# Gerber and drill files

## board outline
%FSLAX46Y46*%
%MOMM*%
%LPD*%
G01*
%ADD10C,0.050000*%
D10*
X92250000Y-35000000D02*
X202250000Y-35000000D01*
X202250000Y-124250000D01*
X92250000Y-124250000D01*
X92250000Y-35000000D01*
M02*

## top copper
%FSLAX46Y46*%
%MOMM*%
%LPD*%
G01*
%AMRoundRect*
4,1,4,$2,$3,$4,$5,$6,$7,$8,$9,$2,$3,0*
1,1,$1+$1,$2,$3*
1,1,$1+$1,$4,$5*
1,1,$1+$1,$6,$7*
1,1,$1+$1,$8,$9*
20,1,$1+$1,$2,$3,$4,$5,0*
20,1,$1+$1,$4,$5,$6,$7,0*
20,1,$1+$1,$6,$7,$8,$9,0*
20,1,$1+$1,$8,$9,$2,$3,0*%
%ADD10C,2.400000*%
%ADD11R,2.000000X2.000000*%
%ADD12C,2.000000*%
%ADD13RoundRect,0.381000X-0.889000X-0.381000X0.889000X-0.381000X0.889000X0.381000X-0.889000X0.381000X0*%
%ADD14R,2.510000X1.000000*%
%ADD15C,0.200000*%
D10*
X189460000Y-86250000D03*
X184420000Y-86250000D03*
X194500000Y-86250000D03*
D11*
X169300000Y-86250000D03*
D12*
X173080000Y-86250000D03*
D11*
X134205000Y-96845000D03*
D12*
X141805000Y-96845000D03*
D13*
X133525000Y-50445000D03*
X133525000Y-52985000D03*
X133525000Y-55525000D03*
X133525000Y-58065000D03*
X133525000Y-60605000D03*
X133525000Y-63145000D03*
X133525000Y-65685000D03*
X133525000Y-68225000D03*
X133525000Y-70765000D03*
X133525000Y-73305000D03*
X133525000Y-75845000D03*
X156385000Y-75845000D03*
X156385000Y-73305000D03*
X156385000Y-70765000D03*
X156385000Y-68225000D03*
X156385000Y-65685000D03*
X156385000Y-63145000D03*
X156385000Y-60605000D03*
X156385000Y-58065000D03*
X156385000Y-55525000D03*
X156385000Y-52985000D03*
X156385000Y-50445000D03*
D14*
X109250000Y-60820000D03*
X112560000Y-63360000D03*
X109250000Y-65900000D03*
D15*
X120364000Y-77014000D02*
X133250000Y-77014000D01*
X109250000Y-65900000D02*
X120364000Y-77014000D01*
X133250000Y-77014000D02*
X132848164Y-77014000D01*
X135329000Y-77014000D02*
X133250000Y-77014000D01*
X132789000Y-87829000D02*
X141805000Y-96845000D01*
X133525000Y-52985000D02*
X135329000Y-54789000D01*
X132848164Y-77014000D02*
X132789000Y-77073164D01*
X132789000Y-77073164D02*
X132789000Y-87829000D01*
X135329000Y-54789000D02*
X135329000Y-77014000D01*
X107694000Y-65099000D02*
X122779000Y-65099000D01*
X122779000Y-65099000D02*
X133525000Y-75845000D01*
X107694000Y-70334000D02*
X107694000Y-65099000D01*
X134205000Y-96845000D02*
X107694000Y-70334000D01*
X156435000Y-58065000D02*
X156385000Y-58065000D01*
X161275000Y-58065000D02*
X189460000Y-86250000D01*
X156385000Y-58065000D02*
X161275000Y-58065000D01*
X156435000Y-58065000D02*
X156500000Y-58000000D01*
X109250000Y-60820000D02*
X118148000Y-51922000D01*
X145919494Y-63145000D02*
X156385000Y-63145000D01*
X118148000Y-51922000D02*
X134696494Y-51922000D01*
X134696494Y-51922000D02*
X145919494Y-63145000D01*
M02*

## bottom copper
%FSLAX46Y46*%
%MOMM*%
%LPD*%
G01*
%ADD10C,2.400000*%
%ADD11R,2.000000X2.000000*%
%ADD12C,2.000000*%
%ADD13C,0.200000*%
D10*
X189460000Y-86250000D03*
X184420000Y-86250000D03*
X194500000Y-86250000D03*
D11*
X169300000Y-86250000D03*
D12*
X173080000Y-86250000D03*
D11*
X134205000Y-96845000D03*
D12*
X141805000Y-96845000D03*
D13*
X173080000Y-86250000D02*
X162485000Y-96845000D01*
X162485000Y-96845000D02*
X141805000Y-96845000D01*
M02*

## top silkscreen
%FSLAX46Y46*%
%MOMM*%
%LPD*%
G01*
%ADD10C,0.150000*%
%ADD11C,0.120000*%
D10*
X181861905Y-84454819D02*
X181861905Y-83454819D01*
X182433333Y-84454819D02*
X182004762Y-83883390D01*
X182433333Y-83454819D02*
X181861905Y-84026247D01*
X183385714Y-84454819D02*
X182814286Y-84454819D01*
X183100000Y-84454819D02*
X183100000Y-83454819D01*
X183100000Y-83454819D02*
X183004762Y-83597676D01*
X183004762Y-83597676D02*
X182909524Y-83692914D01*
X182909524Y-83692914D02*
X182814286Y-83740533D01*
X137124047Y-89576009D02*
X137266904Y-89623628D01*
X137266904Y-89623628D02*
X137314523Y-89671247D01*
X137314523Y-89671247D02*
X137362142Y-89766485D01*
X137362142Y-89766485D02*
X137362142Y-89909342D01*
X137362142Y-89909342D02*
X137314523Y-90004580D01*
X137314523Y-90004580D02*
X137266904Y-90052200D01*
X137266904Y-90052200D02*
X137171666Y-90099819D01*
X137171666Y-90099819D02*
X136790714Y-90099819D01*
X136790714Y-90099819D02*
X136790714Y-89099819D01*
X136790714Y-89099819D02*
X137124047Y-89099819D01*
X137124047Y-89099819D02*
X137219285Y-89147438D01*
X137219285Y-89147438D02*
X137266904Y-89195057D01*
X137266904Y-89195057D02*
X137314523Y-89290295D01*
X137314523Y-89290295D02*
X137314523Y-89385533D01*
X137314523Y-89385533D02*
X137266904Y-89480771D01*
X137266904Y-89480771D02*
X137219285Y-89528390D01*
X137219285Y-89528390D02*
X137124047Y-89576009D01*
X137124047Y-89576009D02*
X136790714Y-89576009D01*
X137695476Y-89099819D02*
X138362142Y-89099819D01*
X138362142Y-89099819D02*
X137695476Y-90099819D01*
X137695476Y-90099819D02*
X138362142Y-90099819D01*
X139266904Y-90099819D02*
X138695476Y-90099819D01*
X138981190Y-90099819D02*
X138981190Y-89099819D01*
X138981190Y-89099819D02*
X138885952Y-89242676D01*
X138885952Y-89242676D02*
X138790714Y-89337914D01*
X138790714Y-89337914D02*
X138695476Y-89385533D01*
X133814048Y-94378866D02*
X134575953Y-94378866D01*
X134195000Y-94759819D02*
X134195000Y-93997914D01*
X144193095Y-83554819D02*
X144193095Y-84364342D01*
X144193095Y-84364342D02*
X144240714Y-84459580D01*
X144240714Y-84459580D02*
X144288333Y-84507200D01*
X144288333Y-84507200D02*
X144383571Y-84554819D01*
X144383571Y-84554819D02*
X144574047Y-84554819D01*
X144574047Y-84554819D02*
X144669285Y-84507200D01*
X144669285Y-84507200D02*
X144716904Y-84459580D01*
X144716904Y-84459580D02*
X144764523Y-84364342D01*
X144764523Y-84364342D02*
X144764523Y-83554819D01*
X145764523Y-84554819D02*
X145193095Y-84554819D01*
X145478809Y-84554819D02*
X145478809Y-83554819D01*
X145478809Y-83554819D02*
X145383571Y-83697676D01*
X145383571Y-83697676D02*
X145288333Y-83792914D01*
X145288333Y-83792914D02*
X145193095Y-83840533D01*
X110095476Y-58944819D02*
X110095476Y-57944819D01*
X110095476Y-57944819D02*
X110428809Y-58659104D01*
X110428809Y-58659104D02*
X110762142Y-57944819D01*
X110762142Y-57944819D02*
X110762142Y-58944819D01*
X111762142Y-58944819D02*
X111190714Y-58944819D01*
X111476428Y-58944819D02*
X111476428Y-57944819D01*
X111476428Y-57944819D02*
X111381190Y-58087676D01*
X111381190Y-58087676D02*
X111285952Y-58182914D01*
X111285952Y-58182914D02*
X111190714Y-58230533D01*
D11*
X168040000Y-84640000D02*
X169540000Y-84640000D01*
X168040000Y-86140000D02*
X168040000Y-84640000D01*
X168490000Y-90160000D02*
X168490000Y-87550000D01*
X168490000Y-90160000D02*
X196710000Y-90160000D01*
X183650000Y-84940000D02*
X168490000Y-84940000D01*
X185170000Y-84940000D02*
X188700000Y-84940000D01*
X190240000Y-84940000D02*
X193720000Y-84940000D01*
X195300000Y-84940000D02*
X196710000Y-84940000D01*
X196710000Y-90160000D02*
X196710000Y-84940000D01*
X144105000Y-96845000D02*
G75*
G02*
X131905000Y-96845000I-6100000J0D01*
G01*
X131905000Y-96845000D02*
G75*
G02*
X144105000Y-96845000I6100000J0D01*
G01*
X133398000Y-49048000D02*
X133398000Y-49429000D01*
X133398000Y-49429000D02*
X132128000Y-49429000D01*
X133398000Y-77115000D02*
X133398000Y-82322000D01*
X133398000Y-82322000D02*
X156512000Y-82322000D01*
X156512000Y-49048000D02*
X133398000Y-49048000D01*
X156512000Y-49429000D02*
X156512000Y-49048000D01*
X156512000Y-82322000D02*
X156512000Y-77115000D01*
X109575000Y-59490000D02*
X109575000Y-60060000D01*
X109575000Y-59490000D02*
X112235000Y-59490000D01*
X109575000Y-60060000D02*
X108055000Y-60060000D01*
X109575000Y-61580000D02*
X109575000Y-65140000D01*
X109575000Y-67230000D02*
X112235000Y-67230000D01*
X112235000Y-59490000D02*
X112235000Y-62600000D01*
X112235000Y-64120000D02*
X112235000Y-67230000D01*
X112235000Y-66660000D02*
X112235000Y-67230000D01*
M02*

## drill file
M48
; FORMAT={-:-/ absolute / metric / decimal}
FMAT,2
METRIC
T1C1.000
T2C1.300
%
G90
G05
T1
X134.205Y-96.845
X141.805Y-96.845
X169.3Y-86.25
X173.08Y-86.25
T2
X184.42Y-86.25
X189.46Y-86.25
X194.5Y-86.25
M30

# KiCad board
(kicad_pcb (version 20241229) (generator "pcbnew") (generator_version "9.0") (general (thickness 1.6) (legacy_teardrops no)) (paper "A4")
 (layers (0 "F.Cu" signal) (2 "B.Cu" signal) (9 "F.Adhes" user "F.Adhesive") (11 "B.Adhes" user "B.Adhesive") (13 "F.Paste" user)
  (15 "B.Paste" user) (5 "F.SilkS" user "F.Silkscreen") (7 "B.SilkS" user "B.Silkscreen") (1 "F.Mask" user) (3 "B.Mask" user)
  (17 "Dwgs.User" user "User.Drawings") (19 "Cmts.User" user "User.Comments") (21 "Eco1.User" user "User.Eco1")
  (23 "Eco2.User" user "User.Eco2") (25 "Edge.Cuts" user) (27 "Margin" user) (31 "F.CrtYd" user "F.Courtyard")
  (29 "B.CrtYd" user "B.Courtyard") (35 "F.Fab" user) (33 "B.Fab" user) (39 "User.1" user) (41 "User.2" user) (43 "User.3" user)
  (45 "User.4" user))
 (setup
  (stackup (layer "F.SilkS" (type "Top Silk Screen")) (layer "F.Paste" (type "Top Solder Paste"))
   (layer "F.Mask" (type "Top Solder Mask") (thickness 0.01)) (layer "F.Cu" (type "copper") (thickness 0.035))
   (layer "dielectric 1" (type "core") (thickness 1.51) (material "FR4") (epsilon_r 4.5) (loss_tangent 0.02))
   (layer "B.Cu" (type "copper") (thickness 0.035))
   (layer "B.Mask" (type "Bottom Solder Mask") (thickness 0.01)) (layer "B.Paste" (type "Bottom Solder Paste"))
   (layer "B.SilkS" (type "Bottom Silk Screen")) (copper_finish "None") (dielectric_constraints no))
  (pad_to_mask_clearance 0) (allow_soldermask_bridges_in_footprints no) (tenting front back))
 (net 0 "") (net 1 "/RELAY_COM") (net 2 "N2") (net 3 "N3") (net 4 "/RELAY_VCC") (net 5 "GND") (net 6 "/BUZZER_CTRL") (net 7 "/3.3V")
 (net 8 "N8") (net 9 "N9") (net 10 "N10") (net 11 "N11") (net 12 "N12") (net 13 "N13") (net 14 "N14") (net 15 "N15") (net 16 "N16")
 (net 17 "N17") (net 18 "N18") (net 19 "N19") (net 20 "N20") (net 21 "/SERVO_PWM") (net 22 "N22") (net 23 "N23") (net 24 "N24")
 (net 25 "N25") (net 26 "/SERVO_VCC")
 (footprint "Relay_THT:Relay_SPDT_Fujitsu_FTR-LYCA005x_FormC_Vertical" (layer "F.Cu") (at 169.3 86.25)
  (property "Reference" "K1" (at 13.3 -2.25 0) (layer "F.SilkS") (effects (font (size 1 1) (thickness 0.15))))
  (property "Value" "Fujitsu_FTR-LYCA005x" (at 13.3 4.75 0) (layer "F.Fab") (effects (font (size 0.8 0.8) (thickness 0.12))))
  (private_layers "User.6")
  (fp_line (start -1.26 -1.61) (end 0.24 -1.61) (stroke (width 0.12) (type solid)) (layer "F.SilkS"))
  (fp_line (start -1.26 -0.11) (end -1.26 -1.61) (stroke (width 0.12) (type solid)) (layer "F.SilkS"))
  (fp_line (start -0.81 3.91) (end -0.81 1.3) (stroke (width 0.12) (type solid)) (layer "F.SilkS"))
  (fp_line (start -0.81 3.91) (end 27.41 3.91) (stroke (width 0.12) (type solid)) (layer "F.SilkS"))
  (fp_line (start 14.35 -1.31) (end -0.81 -1.31) (stroke (width 0.12) (type solid)) (layer "F.SilkS"))
  (fp_line (start 15.87 -1.31) (end 19.4 -1.31) (stroke (width 0.12) (type solid)) (layer "F.SilkS"))
  (fp_line (start 20.94 -1.31) (end 24.42 -1.31) (stroke (width 0.12) (type solid)) (layer "F.SilkS"))
  (fp_line (start 26 -1.31) (end 27.41 -1.31) (stroke (width 0.12) (type solid)) (layer "F.SilkS"))
  (fp_line (start 27.41 3.91) (end 27.41 -1.31) (stroke (width 0.12) (type solid)) (layer "F.SilkS"))
  (pad "11" thru_hole circle (at 20.16 0) (size 2.4 2.4) (drill 1.3) (layers "*.Cu" "*.Mask") (remove_unused_layers no) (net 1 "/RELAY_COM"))
  (pad "12" thru_hole circle (at 15.12 0) (size 2.4 2.4) (drill 1.3) (layers "*.Cu" "*.Mask") (remove_unused_layers no) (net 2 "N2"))
  (pad "14" thru_hole circle (at 25.2 0) (size 2.4 2.4) (drill 1.3) (layers "*.Cu" "*.Mask") (remove_unused_layers no) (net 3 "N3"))
  (pad "A1" thru_hole rect (at 0 0) (size 2 2) (drill 1) (layers "*.Cu" "*.Mask") (remove_unused_layers no) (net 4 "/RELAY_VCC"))
  (pad "A2" thru_hole circle (at 3.78 0) (size 2 2) (drill 1) (layers "*.Cu" "*.Mask") (remove_unused_layers no) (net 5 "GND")))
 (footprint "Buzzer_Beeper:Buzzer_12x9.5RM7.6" (layer "F.Cu") (at 134.205 96.845)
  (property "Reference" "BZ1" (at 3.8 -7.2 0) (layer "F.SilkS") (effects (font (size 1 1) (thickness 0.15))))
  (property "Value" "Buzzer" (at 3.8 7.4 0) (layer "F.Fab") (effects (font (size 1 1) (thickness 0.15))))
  (fp_circle (center 3.8 0) (end 9.9 0) (stroke (width 0.12) (type solid)) (fill no) (layer "F.SilkS"))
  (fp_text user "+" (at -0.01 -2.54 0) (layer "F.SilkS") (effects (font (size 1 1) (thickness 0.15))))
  (pad "1" thru_hole rect (at 0 0) (size 2 2) (drill 1) (layers "*.Cu" "*.Mask") (remove_unused_layers no) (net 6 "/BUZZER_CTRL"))
  (pad "2" thru_hole circle (at 7.6 0) (size 2 2) (drill 1) (layers "*.Cu" "*.Mask") (remove_unused_layers no) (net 5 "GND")))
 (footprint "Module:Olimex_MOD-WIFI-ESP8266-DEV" (layer "F.Cu") (at 144.955 63.145)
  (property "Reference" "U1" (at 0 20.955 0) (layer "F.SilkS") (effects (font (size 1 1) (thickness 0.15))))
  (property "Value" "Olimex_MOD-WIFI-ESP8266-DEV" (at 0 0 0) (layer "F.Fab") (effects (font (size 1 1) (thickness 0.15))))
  (fp_line (start -11.557 -14.097) (end -11.557 -13.716) (stroke (width 0.12) (type solid)) (layer "F.SilkS"))
  (fp_line (start -11.557 -13.716) (end -12.827 -13.716) (stroke (width 0.12) (type solid)) (layer "F.SilkS"))
  (fp_line (start -11.557 13.97) (end -11.557 19.177) (stroke (width 0.12) (type solid)) (layer "F.SilkS"))
  (fp_line (start -11.557 19.177) (end 11.557 19.177) (stroke (width 0.12) (type solid)) (layer "F.SilkS"))
  (fp_line (start 11.557 -14.097) (end -11.557 -14.097) (stroke (width 0.12) (type solid)) (layer "F.SilkS"))
  (fp_line (start 11.557 -13.716) (end 11.557 -14.097) (stroke (width 0.12) (type solid)) (layer "F.SilkS"))
  (fp_line (start 11.557 19.177) (end 11.557 13.97) (stroke (width 0.12) (type solid)) (layer "F.SilkS"))
  (pad "1" smd roundrect (at -11.43 -12.7) (size 2.54 1.524) (layers "F.Cu" "F.Mask" "F.Paste") (roundrect_rratio 0.25) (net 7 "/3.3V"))
  (pad "2" smd roundrect (at -11.43 -10.16) (size 2.54 1.524) (layers "F.Cu" "F.Mask" "F.Paste") (roundrect_rratio 0.25) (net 5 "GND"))
  (pad "3" smd roundrect (at -11.43 -7.62) (size 2.54 1.524) (layers "F.Cu" "F.Mask" "F.Paste") (roundrect_rratio 0.25) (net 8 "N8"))
  (pad "4" smd roundrect (at -11.43 -5.08) (size 2.54 1.524) (layers "F.Cu" "F.Mask" "F.Paste") (roundrect_rratio 0.25) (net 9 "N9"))
  (pad "5" smd roundrect (at -11.43 -2.54) (size 2.54 1.524) (layers "F.Cu" "F.Mask" "F.Paste") (roundrect_rratio 0.25) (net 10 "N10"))
  (pad "6" smd roundrect (at -11.43 0) (size 2.54 1.524) (layers "F.Cu" "F.Mask" "F.Paste") (roundrect_rratio 0.25) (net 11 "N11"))
  (pad "7" smd roundrect (at -11.43 2.54) (size 2.54 1.524) (layers "F.Cu" "F.Mask" "F.Paste") (roundrect_rratio 0.25) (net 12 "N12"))
  (pad "8" smd roundrect (at -11.43 5.08) (size 2.54 1.524) (layers "F.Cu" "F.Mask" "F.Paste") (roundrect_rratio 0.25) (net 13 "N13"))
  (pad "9" smd roundrect (at -11.43 7.62) (size 2.54 1.524) (layers "F.Cu" "F.Mask" "F.Paste") (roundrect_rratio 0.25) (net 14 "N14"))
  (pad "10" smd roundrect (at -11.43 10.16) (size 2.54 1.524) (layers "F.Cu" "F.Mask" "F.Paste") (roundrect_rratio 0.25) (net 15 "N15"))
  (pad "11" smd roundrect (at -11.43 12.7) (size 2.54 1.524) (layers "F.Cu" "F.Mask" "F.Paste") (roundrect_rratio 0.25)
   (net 6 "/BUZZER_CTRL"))
  (pad "12" smd roundrect (at 11.43 12.7) (size 2.54 1.524) (layers "F.Cu" "F.Mask" "F.Paste") (roundrect_rratio 0.25) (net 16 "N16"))
  (pad "13" smd roundrect (at 11.43 10.16) (size 2.54 1.524) (layers "F.Cu" "F.Mask" "F.Paste") (roundrect_rratio 0.25) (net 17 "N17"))
  (pad "14" smd roundrect (at 11.43 7.62) (size 2.54 1.524) (layers "F.Cu" "F.Mask" "F.Paste") (roundrect_rratio 0.25) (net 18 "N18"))
  (pad "15" smd roundrect (at 11.43 5.08) (size 2.54 1.524) (layers "F.Cu" "F.Mask" "F.Paste") (roundrect_rratio 0.25) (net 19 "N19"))
  (pad "16" smd roundrect (at 11.43 2.54) (size 2.54 1.524) (layers "F.Cu" "F.Mask" "F.Paste") (roundrect_rratio 0.25) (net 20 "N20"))
  (pad "17" smd roundrect (at 11.43 0) (size 2.54 1.524) (layers "F.Cu" "F.Mask" "F.Paste") (roundrect_rratio 0.25) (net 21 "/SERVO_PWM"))
  (pad "18" smd roundrect (at 11.43 -2.54) (size 2.54 1.524) (layers "F.Cu" "F.Mask" "F.Paste") (roundrect_rratio 0.25) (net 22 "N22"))
  (pad "19" smd roundrect (at 11.43 -5.08) (size 2.54 1.524) (layers "F.Cu" "F.Mask" "F.Paste") (roundrect_rratio 0.25) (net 1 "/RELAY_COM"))
  (pad "20" smd roundrect (at 11.43 -7.62) (size 2.54 1.524) (layers "F.Cu" "F.Mask" "F.Paste") (roundrect_rratio 0.25) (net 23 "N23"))
  (pad "21" smd roundrect (at 11.43 -10.16) (size 2.54 1.524) (layers "F.Cu" "F.Mask" "F.Paste") (roundrect_rratio 0.25) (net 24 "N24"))
  (pad "22" smd roundrect (at 11.43 -12.7) (size 2.54 1.524) (layers "F.Cu" "F.Mask" "F.Paste") (roundrect_rratio 0.25) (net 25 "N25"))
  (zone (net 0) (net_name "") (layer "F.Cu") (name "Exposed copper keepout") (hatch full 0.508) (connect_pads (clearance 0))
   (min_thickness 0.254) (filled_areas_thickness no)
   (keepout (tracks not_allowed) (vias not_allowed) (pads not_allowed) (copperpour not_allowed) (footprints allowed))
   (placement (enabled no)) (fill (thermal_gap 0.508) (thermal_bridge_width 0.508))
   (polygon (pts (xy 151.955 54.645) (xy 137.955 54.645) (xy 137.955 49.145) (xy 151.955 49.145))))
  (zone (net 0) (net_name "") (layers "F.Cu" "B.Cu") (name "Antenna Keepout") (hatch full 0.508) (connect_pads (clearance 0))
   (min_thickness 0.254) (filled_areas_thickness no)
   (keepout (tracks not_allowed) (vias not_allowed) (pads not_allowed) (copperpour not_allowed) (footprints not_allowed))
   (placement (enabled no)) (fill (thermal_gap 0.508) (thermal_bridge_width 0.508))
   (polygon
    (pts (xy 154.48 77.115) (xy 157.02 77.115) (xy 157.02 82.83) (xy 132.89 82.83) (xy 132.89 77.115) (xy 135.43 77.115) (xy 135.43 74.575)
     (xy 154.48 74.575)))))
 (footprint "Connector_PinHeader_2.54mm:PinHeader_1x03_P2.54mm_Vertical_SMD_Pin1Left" (layer "F.Cu") (at 110.905 63.36)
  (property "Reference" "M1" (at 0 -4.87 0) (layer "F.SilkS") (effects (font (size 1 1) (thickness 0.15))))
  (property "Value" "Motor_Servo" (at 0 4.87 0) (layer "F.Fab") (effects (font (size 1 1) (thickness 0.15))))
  (fp_line (start -1.33 -3.87) (end -1.33 -3.3) (stroke (width 0.12) (type solid)) (layer "F.SilkS"))
  (fp_line (start -1.33 -3.87) (end 1.33 -3.87) (stroke (width 0.12) (type solid)) (layer "F.SilkS"))
  (fp_line (start -1.33 -3.3) (end -2.85 -3.3) (stroke (width 0.12) (type solid)) (layer "F.SilkS"))
  (fp_line (start -1.33 -1.78) (end -1.33 1.78) (stroke (width 0.12) (type solid)) (layer "F.SilkS"))
  (fp_line (start -1.33 3.87) (end 1.33 3.87) (stroke (width 0.12) (type solid)) (layer "F.SilkS"))
  (fp_line (start 1.33 -3.87) (end 1.33 -0.76) (stroke (width 0.12) (type solid)) (layer "F.SilkS"))
  (fp_line (start 1.33 0.76) (end 1.33 3.87) (stroke (width 0.12) (type solid)) (layer "F.SilkS"))
  (fp_line (start 1.33 3.3) (end 1.33 3.87) (stroke (width 0.12) (type solid)) (layer "F.SilkS"))
  (pad "1" smd rect (at -1.655 -2.54) (size 2.51 1) (layers "F.Cu" "F.Mask" "F.Paste") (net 21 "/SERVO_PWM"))
  (pad "2" smd rect (at 1.655 0) (size 2.51 1) (layers "F.Cu" "F.Mask" "F.Paste") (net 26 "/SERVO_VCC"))
  (pad "3" smd rect (at -1.655 2.54) (size 2.51 1) (layers "F.Cu" "F.Mask" "F.Paste") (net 5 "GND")))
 (gr_rect (start 92.25 35) (end 202.25 124.25) (stroke (width 0.05) (type default)) (fill no) (layer "Edge.Cuts"))
 (segment (start 120.364 77.014) (end 133.25 77.014) (width 0.2) (layer "F.Cu") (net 5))
 (segment (start 109.25 65.9) (end 120.364 77.014) (width 0.2) (layer "F.Cu") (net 5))
 (segment (start 133.25 77.014) (end 132.848164 77.014) (width 0.2) (layer "F.Cu") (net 5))
 (segment (start 135.329 77.014) (end 133.25 77.014) (width 0.2) (layer "F.Cu") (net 5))
 (segment (start 132.789 87.829) (end 141.805 96.845) (width 0.2) (layer "F.Cu") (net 5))
 (segment (start 133.525 52.985) (end 135.329 54.789) (width 0.2) (layer "F.Cu") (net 5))
 (segment (start 132.848164 77.014) (end 132.789 77.073164) (width 0.2) (layer "F.Cu") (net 5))
 (segment (start 132.789 77.073164) (end 132.789 87.829) (width 0.2) (layer "F.Cu") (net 5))
 (segment (start 135.329 54.789) (end 135.329 77.014) (width 0.2) (layer "F.Cu") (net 5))
 (segment (start 173.08 86.25) (end 162.485 96.845) (width 0.2) (layer "B.Cu") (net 5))
 (segment (start 162.485 96.845) (end 141.805 96.845) (width 0.2) (layer "B.Cu") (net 5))
 (segment (start 107.694 65.099) (end 122.779 65.099) (width 0.2) (layer "F.Cu") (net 6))
 (segment (start 122.779 65.099) (end 133.525 75.845) (width 0.2) (layer "F.Cu") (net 6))
 (segment (start 107.694 70.334) (end 107.694 65.099) (width 0.2) (layer "F.Cu") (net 6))
 (segment (start 134.205 96.845) (end 107.694 70.334) (width 0.2) (layer "F.Cu") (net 6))
 (segment (start 156.435 58.065) (end 156.385 58.065) (width 0.2) (layer "F.Cu") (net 1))
 (segment (start 161.275 58.065) (end 189.46 86.25) (width 0.2) (layer "F.Cu") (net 1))
 (segment (start 156.385 58.065) (end 161.275 58.065) (width 0.2) (layer "F.Cu") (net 1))
 (segment (start 156.435 58.065) (end 156.5 58) (width 0.2) (layer "F.Cu") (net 1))
 (segment (start 109.25 60.82) (end 118.148 51.922) (width 0.2) (layer "F.Cu") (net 21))
 (segment (start 145.919494 63.145) (end 156.385 63.145) (width 0.2) (layer "F.Cu") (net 21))
 (segment (start 118.148 51.922) (end 134.696494 51.922) (width 0.2) (layer "F.Cu") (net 21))
 (segment (start 134.696494 51.922) (end 145.919494 63.145) (width 0.2) (layer "F.Cu") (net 21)))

